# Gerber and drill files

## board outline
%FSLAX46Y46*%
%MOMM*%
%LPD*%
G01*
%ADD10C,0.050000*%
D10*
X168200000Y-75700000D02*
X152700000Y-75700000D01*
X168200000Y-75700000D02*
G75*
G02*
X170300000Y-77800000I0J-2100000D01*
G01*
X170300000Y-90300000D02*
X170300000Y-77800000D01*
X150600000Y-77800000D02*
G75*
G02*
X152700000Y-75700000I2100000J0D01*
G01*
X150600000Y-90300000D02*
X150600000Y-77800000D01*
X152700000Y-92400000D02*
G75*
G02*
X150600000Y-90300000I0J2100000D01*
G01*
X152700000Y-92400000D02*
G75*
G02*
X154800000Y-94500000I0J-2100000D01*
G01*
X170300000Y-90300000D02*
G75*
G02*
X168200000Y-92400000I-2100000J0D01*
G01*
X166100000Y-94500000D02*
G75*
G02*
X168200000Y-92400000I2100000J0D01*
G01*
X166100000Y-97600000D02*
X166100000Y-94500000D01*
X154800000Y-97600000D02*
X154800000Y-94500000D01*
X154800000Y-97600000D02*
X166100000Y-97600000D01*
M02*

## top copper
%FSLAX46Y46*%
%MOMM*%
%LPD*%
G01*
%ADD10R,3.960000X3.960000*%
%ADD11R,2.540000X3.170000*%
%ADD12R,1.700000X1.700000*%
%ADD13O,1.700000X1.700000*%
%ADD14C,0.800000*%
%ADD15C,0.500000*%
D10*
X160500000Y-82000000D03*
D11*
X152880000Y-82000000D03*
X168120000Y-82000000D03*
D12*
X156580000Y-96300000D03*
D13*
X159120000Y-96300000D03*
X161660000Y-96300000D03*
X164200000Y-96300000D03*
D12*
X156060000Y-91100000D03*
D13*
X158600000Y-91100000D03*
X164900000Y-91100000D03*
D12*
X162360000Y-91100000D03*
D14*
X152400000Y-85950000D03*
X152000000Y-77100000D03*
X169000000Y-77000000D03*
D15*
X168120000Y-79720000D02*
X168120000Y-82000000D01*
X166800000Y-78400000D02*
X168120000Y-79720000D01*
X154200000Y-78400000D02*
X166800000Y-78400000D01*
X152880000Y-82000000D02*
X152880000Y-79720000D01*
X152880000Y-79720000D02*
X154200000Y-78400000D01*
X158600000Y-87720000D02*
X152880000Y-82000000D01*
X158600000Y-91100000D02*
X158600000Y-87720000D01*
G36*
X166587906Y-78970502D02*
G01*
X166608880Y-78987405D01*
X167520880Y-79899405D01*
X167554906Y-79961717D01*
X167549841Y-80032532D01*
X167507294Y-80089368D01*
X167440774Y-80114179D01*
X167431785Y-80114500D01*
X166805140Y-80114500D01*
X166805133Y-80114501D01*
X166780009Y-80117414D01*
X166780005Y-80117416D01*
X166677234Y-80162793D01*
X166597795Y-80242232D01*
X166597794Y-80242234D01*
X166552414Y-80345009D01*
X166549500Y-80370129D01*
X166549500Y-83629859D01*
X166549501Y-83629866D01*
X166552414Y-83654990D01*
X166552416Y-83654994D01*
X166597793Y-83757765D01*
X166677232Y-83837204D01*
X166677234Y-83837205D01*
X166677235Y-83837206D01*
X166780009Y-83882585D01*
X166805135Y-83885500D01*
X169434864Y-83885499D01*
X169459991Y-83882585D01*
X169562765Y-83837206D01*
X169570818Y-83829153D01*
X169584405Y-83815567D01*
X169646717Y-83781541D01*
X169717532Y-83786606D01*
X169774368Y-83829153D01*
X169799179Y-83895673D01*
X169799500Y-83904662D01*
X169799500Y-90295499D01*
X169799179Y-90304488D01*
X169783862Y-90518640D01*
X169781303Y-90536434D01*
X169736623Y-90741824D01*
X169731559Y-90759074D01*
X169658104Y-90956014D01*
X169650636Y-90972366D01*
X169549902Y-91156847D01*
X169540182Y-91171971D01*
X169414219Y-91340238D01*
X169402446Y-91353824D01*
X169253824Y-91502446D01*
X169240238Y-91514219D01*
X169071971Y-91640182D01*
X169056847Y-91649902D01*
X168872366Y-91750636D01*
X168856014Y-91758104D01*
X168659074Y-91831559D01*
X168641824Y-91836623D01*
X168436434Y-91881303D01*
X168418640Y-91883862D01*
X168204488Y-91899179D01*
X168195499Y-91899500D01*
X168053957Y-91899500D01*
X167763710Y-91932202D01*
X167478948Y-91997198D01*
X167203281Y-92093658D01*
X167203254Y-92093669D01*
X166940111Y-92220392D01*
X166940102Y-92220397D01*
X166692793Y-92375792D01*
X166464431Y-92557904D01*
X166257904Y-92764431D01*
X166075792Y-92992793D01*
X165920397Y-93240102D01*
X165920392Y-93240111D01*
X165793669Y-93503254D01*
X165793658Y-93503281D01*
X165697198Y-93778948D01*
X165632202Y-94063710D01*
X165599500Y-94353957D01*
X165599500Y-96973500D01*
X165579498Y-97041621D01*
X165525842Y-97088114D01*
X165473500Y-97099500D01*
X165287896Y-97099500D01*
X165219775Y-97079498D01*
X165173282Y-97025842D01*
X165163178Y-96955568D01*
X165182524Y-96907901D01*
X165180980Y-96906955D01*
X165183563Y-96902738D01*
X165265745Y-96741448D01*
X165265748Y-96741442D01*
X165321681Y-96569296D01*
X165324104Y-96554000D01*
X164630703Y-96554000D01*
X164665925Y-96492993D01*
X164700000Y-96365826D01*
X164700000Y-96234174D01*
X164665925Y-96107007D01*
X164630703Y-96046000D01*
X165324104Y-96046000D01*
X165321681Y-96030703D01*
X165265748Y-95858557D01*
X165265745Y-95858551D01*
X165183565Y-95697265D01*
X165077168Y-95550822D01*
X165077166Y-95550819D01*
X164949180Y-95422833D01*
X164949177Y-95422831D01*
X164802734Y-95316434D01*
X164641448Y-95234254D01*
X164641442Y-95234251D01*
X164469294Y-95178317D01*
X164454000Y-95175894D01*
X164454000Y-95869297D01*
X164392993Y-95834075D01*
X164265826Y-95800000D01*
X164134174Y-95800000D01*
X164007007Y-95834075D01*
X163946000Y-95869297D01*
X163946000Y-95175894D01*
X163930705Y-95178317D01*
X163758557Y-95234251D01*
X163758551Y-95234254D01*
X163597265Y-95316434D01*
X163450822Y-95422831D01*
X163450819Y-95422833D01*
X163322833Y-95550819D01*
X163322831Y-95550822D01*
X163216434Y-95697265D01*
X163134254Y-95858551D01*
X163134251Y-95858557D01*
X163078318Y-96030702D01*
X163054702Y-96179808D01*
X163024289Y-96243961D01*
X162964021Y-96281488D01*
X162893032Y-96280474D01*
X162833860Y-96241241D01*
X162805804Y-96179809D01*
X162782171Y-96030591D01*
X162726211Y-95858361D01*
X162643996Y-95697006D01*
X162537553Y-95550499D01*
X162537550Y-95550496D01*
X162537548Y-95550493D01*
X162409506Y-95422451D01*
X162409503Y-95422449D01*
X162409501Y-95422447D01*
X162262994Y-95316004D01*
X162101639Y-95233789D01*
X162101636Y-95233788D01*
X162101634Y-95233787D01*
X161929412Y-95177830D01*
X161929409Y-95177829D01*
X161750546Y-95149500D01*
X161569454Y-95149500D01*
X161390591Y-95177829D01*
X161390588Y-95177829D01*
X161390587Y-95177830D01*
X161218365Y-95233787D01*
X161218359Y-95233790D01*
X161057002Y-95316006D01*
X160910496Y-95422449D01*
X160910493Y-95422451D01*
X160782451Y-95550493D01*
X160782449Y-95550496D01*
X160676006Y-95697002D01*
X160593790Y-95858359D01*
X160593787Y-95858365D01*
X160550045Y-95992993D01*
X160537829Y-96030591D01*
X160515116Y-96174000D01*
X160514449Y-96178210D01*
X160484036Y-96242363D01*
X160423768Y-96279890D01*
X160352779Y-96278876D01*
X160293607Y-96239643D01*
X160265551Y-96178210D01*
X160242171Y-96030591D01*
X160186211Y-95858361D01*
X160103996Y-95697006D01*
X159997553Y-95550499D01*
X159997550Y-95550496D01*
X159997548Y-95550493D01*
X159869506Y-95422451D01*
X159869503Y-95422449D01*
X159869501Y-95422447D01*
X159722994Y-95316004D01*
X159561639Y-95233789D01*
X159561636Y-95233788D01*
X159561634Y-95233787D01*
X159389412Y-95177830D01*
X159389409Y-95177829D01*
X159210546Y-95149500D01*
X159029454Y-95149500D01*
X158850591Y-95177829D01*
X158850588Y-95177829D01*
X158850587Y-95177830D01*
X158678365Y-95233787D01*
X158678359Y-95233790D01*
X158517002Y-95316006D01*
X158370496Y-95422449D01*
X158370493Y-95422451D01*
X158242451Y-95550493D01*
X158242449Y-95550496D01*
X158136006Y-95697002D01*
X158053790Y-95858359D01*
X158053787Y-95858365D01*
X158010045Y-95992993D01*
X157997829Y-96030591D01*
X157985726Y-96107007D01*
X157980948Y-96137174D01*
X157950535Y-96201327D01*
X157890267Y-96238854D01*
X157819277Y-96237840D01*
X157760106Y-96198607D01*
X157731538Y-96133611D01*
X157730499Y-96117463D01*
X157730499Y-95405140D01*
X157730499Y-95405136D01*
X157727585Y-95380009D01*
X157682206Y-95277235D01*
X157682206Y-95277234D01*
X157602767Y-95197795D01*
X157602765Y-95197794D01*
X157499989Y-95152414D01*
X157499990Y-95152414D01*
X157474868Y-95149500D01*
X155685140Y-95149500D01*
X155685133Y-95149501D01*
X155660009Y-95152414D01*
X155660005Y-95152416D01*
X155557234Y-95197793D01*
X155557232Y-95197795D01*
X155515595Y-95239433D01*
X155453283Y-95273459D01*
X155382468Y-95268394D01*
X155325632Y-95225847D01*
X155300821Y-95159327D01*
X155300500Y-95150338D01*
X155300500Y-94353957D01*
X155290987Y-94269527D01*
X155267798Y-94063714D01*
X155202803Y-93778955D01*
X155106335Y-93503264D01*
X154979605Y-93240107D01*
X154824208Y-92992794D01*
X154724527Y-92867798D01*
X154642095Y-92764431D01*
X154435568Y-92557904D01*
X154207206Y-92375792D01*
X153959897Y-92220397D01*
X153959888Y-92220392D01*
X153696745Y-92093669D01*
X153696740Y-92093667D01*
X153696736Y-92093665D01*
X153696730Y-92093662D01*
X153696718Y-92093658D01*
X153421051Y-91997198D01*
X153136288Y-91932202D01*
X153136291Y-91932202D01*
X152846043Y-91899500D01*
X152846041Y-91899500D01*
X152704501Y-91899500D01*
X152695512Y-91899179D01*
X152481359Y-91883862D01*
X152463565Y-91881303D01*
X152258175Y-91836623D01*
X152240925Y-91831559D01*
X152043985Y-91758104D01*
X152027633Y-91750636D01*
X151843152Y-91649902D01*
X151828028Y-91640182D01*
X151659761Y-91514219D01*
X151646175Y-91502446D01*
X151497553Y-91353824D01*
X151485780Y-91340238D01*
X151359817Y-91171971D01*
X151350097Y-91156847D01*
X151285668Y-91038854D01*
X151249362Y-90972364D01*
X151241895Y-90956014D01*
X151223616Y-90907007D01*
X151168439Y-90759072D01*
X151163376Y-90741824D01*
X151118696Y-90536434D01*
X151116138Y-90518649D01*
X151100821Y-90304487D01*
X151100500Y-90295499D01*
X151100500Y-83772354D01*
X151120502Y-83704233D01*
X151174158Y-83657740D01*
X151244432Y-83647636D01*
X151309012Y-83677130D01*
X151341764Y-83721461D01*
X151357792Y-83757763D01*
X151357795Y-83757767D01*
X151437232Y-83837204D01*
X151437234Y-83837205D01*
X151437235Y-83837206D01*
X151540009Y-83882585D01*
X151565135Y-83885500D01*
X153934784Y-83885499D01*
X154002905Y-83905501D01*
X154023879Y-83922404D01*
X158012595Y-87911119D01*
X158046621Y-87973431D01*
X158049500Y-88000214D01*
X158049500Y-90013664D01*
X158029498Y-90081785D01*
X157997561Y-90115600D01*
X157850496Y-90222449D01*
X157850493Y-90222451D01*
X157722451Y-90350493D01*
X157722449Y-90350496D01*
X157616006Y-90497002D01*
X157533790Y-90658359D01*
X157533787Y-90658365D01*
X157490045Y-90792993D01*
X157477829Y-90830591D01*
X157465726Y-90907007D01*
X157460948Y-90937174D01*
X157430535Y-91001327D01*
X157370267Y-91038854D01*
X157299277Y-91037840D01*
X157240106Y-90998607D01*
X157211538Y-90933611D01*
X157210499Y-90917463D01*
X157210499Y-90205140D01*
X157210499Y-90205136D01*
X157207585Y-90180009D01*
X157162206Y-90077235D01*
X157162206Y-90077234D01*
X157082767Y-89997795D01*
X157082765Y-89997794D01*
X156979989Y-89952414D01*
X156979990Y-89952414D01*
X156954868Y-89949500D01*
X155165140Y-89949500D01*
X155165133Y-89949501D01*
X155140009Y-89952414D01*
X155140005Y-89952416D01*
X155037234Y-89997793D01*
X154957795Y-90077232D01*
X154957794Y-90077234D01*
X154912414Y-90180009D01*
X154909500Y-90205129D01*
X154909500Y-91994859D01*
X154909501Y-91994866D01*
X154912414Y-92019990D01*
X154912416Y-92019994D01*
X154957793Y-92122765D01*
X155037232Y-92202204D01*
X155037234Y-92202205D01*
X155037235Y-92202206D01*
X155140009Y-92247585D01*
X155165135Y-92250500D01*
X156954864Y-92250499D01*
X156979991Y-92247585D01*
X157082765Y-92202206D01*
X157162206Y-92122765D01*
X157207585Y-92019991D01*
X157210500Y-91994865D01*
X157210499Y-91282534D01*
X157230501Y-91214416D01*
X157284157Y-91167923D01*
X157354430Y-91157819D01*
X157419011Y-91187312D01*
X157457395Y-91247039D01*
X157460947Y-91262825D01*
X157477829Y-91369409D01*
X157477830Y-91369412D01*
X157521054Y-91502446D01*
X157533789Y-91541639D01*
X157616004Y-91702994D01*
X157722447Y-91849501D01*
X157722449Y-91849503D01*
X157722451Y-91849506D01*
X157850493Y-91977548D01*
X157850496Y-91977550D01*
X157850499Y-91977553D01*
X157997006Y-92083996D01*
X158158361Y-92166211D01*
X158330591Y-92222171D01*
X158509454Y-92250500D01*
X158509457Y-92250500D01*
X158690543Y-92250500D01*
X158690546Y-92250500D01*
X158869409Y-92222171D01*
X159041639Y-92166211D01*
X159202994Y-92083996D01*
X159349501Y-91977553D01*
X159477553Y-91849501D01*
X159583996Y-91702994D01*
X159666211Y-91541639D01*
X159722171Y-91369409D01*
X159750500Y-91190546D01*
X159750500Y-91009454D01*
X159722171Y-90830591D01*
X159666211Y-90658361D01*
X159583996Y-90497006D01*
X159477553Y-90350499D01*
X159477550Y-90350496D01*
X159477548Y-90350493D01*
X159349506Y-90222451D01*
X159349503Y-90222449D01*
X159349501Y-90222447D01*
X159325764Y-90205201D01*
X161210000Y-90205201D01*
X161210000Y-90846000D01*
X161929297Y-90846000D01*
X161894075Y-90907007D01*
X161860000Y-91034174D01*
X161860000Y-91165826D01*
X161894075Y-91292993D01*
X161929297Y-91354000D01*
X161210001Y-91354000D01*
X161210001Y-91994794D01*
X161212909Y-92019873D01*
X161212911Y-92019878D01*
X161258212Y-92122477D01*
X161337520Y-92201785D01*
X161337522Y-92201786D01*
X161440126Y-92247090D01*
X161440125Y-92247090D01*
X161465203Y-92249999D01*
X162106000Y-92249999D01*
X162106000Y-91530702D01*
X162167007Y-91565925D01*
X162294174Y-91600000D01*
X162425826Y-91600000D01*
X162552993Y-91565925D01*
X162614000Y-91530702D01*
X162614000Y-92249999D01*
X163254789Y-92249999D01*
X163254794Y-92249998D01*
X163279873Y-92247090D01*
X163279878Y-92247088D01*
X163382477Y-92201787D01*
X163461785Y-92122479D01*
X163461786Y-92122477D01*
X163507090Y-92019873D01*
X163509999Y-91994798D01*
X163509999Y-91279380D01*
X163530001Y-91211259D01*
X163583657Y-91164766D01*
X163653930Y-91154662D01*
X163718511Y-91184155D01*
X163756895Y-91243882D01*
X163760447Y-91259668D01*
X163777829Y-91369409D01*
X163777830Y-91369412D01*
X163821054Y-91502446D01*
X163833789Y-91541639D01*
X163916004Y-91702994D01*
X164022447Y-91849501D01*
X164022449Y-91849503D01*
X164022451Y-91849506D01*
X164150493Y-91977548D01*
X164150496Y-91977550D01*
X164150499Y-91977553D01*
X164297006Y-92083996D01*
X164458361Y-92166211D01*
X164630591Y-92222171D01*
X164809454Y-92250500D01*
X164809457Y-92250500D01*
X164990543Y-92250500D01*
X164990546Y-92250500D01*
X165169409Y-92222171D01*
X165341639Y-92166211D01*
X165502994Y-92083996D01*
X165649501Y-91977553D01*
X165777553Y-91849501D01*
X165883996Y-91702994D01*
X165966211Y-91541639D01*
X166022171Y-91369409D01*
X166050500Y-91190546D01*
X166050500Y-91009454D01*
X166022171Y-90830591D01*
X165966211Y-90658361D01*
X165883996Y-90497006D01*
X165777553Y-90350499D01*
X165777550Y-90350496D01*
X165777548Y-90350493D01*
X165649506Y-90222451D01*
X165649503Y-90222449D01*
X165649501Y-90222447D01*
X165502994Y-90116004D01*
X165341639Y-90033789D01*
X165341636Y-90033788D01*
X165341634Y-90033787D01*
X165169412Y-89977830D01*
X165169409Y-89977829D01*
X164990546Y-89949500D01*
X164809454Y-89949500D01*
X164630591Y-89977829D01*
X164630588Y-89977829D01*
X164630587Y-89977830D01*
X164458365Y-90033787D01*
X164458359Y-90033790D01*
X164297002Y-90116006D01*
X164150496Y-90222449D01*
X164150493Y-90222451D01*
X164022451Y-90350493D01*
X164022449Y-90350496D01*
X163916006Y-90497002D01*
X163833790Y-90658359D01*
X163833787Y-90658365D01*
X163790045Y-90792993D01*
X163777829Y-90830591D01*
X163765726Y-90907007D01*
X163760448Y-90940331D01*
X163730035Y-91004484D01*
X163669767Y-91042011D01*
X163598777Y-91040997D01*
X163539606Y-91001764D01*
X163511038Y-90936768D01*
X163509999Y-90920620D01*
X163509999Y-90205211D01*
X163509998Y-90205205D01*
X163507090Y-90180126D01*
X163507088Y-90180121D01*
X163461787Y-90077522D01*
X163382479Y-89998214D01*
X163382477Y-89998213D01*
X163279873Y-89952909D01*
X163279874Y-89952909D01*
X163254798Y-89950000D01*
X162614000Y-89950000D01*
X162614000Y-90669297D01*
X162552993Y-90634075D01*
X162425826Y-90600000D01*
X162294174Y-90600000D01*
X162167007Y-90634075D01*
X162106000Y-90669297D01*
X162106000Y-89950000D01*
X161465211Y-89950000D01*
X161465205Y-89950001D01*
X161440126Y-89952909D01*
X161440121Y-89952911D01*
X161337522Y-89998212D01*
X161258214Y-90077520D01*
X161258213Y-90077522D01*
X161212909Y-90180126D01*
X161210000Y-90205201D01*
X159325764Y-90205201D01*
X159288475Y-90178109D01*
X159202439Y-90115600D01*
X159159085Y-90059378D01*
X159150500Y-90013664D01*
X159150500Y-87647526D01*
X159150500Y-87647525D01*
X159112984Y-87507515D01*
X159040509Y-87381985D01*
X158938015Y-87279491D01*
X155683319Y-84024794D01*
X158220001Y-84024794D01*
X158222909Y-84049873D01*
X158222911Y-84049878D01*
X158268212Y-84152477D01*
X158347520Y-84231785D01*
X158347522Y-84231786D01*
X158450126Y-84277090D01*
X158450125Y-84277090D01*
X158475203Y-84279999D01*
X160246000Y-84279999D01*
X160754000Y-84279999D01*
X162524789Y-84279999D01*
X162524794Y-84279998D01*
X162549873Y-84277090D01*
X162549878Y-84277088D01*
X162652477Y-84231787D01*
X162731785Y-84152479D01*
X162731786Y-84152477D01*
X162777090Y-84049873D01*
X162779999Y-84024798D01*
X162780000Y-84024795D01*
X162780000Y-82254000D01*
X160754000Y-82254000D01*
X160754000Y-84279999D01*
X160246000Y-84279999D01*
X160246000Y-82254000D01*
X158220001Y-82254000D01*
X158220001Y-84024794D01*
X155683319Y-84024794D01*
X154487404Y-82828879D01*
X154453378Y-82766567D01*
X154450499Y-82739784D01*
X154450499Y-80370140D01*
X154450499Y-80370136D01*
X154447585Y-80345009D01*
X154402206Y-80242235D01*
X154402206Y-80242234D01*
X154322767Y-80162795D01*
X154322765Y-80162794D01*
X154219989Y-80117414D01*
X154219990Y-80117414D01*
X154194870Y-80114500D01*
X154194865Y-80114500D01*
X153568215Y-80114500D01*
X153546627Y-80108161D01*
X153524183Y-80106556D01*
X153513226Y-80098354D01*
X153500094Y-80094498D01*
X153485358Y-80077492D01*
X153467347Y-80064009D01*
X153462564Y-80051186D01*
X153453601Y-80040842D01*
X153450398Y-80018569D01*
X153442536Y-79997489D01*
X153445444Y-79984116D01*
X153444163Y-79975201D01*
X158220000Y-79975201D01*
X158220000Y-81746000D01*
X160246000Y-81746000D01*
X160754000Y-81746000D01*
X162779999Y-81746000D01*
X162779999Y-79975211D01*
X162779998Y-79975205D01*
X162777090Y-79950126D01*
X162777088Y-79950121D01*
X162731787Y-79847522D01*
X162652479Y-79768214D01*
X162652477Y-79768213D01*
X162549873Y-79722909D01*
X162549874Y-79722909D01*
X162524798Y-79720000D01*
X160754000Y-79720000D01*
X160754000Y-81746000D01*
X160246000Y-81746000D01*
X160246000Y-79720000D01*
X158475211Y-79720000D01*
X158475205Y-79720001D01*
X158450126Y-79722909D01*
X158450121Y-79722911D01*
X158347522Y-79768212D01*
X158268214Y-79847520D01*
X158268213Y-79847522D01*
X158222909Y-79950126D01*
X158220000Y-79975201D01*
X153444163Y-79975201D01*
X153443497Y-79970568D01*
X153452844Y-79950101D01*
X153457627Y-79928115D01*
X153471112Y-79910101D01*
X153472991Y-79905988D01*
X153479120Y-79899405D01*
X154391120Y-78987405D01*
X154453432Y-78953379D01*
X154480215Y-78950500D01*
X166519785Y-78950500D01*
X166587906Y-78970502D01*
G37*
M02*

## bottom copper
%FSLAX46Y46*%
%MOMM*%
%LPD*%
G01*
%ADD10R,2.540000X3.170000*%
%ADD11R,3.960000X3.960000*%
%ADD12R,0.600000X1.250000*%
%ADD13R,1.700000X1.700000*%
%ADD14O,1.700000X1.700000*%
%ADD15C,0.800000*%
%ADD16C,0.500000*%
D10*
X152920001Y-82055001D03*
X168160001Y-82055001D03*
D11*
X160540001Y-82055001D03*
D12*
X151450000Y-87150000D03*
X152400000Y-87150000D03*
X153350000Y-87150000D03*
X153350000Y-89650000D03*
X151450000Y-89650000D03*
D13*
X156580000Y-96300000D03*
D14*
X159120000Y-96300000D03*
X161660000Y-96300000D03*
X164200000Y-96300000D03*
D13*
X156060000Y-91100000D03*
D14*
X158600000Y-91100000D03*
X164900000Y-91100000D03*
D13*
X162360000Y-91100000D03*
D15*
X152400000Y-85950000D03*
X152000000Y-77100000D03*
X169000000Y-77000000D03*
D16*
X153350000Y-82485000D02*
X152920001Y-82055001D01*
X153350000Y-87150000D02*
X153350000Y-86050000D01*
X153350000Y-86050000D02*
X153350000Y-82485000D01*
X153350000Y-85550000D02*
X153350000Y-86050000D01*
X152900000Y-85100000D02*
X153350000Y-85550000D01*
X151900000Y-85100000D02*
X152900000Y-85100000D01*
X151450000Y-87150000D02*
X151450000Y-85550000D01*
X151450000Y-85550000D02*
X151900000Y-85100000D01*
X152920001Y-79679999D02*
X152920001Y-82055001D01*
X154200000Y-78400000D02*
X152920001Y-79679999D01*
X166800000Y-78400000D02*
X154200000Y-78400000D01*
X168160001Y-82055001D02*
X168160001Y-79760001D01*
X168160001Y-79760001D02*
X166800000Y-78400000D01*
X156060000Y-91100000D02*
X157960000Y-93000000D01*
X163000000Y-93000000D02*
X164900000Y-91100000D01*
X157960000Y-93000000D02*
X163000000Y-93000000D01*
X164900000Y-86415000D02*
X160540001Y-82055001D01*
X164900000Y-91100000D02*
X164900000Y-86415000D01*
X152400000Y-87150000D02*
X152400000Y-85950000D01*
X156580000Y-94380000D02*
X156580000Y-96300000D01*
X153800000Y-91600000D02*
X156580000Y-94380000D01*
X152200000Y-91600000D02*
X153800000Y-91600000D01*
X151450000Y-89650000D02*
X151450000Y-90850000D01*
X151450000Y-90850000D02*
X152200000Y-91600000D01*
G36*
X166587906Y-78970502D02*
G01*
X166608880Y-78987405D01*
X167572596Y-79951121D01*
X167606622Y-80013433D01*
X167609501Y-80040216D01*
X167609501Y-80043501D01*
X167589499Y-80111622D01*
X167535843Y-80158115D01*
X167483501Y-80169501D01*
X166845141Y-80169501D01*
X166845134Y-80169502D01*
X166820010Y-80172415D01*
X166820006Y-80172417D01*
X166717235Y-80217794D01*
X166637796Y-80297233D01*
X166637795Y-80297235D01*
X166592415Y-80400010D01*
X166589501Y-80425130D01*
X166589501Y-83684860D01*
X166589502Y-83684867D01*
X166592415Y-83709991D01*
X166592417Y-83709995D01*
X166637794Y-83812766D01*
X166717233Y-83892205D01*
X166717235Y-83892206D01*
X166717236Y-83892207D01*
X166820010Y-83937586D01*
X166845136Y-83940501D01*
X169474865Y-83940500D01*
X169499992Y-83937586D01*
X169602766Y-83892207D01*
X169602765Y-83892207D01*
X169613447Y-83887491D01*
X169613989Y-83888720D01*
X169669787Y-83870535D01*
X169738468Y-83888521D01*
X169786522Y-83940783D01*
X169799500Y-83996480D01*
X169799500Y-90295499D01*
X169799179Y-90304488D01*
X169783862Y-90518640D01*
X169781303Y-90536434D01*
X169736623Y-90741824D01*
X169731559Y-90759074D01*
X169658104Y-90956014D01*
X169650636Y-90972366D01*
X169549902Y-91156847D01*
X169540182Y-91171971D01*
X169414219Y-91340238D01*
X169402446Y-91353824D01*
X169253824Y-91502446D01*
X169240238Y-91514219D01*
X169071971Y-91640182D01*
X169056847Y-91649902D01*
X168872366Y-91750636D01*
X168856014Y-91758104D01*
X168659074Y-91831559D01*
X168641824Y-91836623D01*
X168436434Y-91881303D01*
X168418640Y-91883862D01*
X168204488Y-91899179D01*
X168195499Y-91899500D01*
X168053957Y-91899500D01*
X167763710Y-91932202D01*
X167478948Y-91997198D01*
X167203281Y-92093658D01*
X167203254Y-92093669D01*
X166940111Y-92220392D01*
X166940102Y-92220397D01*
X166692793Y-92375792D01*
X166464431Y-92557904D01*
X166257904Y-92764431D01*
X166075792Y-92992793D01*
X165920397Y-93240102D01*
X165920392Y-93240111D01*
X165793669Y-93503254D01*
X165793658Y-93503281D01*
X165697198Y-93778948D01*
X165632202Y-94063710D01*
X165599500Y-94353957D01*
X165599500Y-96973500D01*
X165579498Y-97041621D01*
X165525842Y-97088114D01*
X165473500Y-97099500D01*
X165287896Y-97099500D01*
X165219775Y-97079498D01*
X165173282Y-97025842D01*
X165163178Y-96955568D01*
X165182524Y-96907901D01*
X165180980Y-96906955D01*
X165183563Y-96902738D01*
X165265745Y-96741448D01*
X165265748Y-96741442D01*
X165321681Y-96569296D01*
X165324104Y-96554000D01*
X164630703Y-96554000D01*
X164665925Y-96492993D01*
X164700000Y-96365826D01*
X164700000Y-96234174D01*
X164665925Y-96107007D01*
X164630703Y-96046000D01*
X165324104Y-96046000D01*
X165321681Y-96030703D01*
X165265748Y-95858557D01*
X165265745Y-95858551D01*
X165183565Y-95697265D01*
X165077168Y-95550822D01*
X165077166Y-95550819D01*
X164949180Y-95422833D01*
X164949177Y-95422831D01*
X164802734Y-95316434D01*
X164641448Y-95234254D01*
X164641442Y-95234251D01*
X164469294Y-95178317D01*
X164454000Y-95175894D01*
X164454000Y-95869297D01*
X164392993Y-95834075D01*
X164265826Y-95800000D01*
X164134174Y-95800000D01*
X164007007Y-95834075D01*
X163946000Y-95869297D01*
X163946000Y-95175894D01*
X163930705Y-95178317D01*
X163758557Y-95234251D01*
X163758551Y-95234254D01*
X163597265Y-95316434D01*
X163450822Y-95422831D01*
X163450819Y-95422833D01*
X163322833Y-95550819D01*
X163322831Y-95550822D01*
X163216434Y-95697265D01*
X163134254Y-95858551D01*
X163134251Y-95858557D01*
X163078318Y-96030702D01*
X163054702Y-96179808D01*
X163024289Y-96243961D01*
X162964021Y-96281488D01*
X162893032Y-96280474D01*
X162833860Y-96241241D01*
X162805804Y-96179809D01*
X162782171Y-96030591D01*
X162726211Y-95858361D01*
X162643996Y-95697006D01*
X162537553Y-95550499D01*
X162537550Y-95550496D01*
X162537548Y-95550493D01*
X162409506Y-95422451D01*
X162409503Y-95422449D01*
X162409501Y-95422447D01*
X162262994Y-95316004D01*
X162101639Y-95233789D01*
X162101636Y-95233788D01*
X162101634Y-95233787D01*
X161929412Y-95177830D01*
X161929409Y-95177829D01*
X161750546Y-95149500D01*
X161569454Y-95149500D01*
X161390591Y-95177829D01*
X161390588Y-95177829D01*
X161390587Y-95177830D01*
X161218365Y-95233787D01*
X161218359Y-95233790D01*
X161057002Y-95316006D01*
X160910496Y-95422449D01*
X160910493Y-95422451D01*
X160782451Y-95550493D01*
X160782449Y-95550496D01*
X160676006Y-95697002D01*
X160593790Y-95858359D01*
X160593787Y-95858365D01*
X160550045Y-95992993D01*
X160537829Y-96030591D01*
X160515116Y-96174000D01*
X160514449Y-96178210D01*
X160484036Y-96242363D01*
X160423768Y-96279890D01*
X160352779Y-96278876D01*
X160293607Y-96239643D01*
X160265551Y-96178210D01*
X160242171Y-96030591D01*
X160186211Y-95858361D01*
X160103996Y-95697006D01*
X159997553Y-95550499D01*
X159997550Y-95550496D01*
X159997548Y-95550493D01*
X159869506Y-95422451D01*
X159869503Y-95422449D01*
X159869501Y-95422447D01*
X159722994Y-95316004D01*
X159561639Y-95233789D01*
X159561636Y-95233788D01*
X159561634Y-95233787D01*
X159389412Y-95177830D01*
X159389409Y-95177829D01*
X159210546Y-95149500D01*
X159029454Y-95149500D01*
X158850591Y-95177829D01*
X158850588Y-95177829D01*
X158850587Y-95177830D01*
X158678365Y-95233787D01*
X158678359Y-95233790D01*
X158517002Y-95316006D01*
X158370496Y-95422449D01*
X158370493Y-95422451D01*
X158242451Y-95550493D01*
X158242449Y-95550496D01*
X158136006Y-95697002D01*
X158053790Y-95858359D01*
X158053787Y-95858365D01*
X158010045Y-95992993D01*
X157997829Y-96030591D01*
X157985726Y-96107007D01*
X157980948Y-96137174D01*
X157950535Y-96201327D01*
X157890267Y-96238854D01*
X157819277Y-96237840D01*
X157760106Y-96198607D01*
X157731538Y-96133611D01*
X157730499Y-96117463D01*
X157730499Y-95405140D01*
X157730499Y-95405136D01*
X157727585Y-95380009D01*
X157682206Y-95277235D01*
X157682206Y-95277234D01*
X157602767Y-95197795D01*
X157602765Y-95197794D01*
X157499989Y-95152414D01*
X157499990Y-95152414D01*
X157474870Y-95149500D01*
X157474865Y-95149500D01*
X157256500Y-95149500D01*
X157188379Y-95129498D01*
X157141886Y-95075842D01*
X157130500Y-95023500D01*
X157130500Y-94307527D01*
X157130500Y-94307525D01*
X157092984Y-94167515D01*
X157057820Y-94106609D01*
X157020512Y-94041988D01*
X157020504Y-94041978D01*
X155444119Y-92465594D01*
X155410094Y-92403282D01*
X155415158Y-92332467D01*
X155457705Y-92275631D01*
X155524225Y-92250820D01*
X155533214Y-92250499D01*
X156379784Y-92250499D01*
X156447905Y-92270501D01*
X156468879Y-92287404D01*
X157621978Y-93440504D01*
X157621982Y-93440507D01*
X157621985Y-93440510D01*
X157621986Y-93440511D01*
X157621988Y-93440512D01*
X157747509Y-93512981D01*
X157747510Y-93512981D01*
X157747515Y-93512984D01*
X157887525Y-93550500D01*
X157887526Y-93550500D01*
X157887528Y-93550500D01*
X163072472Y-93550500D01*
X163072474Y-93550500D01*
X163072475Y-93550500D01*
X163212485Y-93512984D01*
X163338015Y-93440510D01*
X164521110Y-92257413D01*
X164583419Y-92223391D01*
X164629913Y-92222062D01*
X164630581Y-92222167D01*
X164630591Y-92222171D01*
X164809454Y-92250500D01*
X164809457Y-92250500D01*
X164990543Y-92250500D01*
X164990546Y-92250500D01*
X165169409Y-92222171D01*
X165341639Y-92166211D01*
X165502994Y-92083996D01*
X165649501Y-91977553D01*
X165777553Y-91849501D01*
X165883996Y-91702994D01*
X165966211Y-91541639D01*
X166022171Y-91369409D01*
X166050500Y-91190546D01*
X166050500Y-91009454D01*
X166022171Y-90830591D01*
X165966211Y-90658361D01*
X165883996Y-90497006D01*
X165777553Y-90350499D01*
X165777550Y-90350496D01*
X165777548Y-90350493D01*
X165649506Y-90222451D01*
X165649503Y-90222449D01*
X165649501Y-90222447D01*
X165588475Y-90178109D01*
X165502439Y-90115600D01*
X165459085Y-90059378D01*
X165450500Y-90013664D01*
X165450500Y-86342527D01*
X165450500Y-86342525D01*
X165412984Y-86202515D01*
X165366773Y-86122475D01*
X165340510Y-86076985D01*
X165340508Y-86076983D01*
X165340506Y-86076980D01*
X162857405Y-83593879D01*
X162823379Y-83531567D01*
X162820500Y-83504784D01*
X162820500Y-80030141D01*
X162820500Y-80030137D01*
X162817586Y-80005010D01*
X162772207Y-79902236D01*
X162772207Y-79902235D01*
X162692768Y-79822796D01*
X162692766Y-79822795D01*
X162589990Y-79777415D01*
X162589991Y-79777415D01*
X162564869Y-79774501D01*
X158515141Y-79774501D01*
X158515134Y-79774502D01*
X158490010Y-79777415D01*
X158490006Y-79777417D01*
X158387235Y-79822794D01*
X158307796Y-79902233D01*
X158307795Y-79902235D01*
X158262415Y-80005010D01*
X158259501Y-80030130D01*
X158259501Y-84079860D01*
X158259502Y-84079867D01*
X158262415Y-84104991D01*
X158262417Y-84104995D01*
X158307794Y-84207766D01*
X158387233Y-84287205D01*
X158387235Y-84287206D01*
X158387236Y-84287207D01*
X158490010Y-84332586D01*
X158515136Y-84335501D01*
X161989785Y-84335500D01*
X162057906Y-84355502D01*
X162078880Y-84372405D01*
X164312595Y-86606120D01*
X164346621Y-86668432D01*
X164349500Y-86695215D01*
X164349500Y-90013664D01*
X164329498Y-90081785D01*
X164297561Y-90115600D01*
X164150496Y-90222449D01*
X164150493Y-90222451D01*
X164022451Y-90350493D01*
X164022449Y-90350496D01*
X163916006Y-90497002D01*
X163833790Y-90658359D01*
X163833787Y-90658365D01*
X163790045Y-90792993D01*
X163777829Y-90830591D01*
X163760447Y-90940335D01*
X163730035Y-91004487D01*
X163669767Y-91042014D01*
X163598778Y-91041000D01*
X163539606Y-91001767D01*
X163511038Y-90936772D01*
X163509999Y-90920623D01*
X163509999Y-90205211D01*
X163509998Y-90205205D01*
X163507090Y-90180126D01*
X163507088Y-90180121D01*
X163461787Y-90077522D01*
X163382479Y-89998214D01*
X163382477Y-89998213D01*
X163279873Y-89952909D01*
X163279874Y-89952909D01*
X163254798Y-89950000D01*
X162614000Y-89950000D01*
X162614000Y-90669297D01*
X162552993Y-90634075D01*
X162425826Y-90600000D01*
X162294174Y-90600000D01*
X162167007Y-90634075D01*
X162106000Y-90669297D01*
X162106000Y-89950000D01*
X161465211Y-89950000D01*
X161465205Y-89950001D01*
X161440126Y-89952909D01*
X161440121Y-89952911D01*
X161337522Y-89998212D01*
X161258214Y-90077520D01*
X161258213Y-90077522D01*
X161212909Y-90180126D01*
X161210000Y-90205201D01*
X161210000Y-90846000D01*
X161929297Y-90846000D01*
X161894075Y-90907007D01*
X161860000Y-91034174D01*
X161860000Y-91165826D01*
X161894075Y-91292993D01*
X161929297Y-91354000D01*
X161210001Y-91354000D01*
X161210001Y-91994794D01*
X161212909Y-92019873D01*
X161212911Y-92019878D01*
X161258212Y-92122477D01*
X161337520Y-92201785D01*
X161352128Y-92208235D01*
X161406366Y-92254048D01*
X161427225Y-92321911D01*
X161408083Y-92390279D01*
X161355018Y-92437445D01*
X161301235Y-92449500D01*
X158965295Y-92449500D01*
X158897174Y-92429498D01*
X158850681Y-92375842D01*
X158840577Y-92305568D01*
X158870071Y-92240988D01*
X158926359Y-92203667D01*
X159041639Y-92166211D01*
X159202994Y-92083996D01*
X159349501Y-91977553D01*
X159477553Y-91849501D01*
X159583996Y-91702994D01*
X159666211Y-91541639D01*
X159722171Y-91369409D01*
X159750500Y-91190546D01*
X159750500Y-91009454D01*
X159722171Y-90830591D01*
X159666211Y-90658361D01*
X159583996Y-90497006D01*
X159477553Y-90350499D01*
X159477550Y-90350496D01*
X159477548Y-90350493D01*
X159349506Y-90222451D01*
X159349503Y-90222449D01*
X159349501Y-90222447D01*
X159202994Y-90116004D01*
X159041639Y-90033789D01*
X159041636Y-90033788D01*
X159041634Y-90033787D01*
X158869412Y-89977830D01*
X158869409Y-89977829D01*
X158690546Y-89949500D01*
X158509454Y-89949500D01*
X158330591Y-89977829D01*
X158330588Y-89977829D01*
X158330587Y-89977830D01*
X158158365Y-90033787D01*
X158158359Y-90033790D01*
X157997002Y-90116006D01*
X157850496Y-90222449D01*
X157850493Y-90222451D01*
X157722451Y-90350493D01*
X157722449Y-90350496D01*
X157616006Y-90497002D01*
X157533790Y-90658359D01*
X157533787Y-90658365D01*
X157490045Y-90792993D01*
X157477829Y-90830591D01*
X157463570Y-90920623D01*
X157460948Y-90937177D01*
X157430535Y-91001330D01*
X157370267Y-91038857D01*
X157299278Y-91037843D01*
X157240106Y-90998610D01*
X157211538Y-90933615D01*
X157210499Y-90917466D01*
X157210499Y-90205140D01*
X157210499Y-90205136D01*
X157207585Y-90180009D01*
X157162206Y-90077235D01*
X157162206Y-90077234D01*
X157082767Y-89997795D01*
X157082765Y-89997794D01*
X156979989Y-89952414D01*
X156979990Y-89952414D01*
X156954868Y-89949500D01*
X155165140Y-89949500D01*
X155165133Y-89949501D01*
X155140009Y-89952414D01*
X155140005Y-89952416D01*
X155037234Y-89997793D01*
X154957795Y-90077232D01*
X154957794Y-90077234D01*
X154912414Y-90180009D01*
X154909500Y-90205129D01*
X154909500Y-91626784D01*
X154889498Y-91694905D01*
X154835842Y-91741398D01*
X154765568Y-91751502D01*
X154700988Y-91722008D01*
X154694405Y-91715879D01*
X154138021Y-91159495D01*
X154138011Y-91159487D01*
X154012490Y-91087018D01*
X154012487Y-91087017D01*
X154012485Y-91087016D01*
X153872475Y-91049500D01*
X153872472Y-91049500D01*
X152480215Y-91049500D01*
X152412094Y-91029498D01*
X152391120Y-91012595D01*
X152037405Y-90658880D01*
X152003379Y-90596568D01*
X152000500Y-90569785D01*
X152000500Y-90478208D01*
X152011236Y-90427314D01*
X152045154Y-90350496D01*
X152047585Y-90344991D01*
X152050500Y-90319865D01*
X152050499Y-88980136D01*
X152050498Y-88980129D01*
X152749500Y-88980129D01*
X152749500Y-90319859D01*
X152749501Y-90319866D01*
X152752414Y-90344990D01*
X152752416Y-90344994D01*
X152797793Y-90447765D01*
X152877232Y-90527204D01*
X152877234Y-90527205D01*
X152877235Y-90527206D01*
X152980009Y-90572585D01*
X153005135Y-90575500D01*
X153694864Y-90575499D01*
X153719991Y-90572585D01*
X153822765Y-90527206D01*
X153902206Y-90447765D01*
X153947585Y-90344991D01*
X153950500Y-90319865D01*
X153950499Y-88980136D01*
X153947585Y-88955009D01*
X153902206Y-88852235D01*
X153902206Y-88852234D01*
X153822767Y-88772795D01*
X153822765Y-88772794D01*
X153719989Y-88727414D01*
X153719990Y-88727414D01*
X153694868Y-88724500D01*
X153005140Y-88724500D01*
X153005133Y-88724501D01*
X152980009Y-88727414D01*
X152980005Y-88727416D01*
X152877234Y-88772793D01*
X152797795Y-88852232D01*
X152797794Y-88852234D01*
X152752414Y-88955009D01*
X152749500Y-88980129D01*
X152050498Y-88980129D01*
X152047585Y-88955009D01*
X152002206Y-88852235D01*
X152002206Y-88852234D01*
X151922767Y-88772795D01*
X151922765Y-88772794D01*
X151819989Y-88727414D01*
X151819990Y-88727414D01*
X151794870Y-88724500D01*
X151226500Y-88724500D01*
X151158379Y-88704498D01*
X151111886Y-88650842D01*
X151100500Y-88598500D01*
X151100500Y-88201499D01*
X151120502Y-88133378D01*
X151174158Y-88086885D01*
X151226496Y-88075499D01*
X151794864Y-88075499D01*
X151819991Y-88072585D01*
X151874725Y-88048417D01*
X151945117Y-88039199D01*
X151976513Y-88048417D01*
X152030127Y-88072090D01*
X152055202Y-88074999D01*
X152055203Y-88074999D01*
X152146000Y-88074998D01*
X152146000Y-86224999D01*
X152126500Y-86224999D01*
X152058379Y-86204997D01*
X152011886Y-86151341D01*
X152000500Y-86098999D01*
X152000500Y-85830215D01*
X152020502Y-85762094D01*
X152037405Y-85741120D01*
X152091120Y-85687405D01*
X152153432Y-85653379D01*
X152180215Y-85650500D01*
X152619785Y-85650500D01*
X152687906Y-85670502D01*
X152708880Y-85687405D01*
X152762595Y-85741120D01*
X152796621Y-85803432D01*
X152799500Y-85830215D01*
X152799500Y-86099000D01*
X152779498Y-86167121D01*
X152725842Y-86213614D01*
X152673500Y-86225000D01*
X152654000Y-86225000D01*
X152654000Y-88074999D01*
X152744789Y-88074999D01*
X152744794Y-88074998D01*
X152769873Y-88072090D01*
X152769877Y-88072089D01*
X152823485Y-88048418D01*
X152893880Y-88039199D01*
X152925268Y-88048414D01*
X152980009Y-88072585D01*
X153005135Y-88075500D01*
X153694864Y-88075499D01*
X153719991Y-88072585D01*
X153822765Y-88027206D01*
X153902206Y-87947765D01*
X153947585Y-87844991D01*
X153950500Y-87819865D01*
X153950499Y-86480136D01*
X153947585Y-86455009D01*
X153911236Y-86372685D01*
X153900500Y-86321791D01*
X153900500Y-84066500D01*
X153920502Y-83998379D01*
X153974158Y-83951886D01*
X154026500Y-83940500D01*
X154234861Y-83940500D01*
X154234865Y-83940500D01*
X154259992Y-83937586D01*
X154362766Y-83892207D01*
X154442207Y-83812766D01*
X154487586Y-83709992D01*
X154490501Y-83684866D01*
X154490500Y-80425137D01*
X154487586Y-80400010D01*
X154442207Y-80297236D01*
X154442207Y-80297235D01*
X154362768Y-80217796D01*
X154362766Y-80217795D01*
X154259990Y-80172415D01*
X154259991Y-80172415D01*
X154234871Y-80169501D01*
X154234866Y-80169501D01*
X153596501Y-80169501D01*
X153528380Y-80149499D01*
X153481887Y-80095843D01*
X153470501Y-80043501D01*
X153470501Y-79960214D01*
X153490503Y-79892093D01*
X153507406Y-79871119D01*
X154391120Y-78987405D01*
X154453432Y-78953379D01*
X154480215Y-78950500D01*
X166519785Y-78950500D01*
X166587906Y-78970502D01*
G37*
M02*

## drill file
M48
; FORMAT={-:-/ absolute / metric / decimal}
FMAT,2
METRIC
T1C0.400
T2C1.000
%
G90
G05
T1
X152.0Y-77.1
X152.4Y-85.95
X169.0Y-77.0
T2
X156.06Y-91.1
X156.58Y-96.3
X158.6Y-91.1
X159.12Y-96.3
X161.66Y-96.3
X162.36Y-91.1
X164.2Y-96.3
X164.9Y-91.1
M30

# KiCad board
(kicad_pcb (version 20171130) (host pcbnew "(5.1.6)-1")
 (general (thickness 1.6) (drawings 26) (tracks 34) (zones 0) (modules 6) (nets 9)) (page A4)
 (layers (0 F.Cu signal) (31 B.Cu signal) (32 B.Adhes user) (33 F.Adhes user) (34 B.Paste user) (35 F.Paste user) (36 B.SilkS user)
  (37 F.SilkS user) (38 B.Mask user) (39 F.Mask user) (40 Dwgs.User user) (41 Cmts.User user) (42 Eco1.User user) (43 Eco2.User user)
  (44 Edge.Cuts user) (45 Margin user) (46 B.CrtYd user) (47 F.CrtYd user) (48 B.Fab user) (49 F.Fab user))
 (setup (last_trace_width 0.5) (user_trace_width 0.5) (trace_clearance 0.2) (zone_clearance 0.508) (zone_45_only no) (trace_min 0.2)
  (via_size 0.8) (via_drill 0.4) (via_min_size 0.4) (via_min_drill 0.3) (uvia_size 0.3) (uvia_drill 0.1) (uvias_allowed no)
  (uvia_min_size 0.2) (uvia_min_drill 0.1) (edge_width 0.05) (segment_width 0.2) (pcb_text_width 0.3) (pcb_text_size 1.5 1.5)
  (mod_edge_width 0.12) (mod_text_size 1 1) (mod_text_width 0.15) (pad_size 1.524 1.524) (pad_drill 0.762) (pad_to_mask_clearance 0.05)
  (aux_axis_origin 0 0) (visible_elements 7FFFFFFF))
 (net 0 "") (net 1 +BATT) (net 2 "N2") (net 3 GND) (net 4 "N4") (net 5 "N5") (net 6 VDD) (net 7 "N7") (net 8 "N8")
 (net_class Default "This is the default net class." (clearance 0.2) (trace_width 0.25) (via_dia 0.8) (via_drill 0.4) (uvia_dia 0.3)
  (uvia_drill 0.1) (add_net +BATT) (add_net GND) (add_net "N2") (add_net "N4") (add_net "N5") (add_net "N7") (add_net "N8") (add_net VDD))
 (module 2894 (layer B.Cu) (at 160.540001 82.055001)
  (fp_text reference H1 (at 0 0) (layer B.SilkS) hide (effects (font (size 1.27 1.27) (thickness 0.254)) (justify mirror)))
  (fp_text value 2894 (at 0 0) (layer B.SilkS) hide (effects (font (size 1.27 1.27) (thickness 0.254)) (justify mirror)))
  (pad 1 smd rect (at -7.62 0) (size 2.54 3.17) (layers B.Cu B.Paste B.Mask) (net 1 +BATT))
  (pad 2 smd rect (at 7.62 0) (size 2.54 3.17) (layers B.Cu B.Paste B.Mask) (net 1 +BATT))
  (pad MP1 smd rect (at 0 0) (size 3.96 3.96) (layers B.Cu B.Paste B.Mask) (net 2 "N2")))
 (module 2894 (layer F.Cu) (at 160.5 82 180)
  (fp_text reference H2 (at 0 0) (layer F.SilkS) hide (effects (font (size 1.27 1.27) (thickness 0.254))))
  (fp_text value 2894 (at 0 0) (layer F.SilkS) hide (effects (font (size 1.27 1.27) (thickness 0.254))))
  (pad MP1 smd rect (at 0 0 180) (size 3.96 3.96) (layers F.Cu F.Paste F.Mask) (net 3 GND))
  (pad 2 smd rect (at 7.62 0 180) (size 2.54 3.17) (layers F.Cu F.Paste F.Mask) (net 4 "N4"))
  (pad 1 smd rect (at -7.62 0 180) (size 2.54 3.17) (layers F.Cu F.Paste F.Mask) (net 4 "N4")))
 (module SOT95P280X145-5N (layer B.Cu) (at 152.4 88.4 270)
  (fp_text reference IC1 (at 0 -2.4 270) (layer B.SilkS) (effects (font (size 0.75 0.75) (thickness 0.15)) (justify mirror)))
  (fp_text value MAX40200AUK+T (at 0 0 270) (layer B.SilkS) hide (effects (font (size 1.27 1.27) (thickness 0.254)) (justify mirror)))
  (pad 1 smd rect (at -1.25 0.95 180) (size 0.6 1.25) (layers B.Cu B.Paste B.Mask) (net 1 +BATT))
  (pad 2 smd rect (at -1.25 0 180) (size 0.6 1.25) (layers B.Cu B.Paste B.Mask) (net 3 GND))
  (pad 3 smd rect (at -1.25 -0.95 180) (size 0.6 1.25) (layers B.Cu B.Paste B.Mask) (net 1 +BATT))
  (pad 4 smd rect (at 1.25 -0.95 180) (size 0.6 1.25) (layers B.Cu B.Paste B.Mask) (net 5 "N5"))
  (pad 5 smd rect (at 1.25 0.95 180) (size 0.6 1.25) (layers B.Cu B.Paste B.Mask) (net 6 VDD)))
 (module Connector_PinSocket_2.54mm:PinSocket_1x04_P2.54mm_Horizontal (layer F.Cu) (at 156.58 96.3 90)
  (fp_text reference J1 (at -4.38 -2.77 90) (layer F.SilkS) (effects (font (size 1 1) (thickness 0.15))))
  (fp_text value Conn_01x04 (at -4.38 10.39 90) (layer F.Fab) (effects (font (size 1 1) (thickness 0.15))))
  (pad 1 thru_hole rect (at 0 0 90) (size 1.7 1.7) (drill 1) (layers *.Cu *.Mask) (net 6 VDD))
  (pad 2 thru_hole oval (at 0 2.54 90) (size 1.7 1.7) (drill 1) (layers *.Cu *.Mask) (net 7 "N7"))
  (pad 3 thru_hole oval (at 0 5.08 90) (size 1.7 1.7) (drill 1) (layers *.Cu *.Mask) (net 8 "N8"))
  (pad 4 thru_hole oval (at 0 7.62 90) (size 1.7 1.7) (drill 1) (layers *.Cu *.Mask) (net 3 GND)))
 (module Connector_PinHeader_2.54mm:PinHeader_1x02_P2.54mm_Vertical (layer F.Cu) (at 156.06 91.1 90)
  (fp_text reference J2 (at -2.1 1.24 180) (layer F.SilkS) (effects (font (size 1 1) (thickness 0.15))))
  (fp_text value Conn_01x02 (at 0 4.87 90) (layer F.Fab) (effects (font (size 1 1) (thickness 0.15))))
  (pad 1 thru_hole rect (at 0 0 90) (size 1.7 1.7) (drill 1) (layers *.Cu *.Mask) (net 2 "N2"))
  (pad 2 thru_hole oval (at 0 2.54 90) (size 1.7 1.7) (drill 1) (layers *.Cu *.Mask) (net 4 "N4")))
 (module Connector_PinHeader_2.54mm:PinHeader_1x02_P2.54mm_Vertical (layer F.Cu) (at 162.36 91.1 90)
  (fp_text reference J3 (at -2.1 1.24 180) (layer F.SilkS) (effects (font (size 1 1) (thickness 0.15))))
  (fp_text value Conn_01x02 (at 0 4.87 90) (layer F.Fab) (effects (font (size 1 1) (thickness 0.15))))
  (pad 2 thru_hole oval (at 0 2.54 90) (size 1.7 1.7) (drill 1) (layers *.Cu *.Mask) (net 2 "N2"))
  (pad 1 thru_hole rect (at 0 0 90) (size 1.7 1.7) (drill 1) (layers *.Cu *.Mask) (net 3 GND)))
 (gr_line (start 168.2 75.7) (end 152.7 75.7) (layer Edge.Cuts) (width 0.05))
 (gr_arc (start 168.2 77.8) (end 170.3 77.8) (angle -90) (layer Edge.Cuts) (width 0.05))
 (gr_line (start 170.3 90.3) (end 170.3 77.8) (layer Edge.Cuts) (width 0.05))
 (gr_arc (start 152.7 77.8) (end 152.7 75.7) (angle -90) (layer Edge.Cuts) (width 0.05))
 (gr_line (start 150.6 90.3) (end 150.6 77.8) (layer Edge.Cuts) (width 0.05))
 (gr_arc (start 152.7 90.3) (end 150.6 90.3) (angle -90) (layer Edge.Cuts) (width 0.05))
 (gr_arc (start 152.7 94.5) (end 154.8 94.5) (angle -90) (layer Edge.Cuts) (width 0.05))
 (gr_arc (start 168.2 90.3) (end 168.2 92.4) (angle -90) (layer Edge.Cuts) (width 0.05))
 (gr_arc (start 168.2 94.5) (end 168.2 92.4) (angle -90) (layer Edge.Cuts) (width 0.05))
 (gr_line (start 166.1 97.6) (end 166.1 94.5) (layer Edge.Cuts) (width 0.05))
 (gr_line (start 154.8 97.6) (end 154.8 94.5) (layer Edge.Cuts) (width 0.05))
 (gr_line (start 154.8 97.6) (end 166.1 97.6) (layer Edge.Cuts) (width 0.05))
 (segment (start 153.35 82.485) (end 152.920001 82.055001) (width 0.5) (layer B.Cu) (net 1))
 (segment (start 153.35 87.15) (end 153.35 86.05) (width 0.5) (layer B.Cu) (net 1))
 (segment (start 153.35 86.05) (end 153.35 82.485) (width 0.5) (layer B.Cu) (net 1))
 (segment (start 153.35 85.55) (end 153.35 86.05) (width 0.5) (layer B.Cu) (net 1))
 (segment (start 152.9 85.1) (end 153.35 85.55) (width 0.5) (layer B.Cu) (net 1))
 (segment (start 151.9 85.1) (end 152.9 85.1) (width 0.5) (layer B.Cu) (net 1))
 (segment (start 151.45 87.15) (end 151.45 85.55) (width 0.5) (layer B.Cu) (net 1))
 (segment (start 151.45 85.55) (end 151.9 85.1) (width 0.5) (layer B.Cu) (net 1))
 (segment (start 152.920001 79.679999) (end 152.920001 82.055001) (width 0.5) (layer B.Cu) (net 1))
 (segment (start 154.2 78.4) (end 152.920001 79.679999) (width 0.5) (layer B.Cu) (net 1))
 (segment (start 166.8 78.4) (end 154.2 78.4) (width 0.5) (layer B.Cu) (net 1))
 (segment (start 168.160001 82.055001) (end 168.160001 79.760001) (width 0.5) (layer B.Cu) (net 1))
 (segment (start 168.160001 79.760001) (end 166.8 78.4) (width 0.5) (layer B.Cu) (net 1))
 (segment (start 156.06 91.1) (end 157.96 93) (width 0.5) (layer B.Cu) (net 2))
 (segment (start 163 93) (end 164.9 91.1) (width 0.5) (layer B.Cu) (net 2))
 (segment (start 157.96 93) (end 163 93) (width 0.5) (layer B.Cu) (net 2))
 (segment (start 164.9 86.415) (end 160.540001 82.055001) (width 0.5) (layer B.Cu) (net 2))
 (segment (start 164.9 91.1) (end 164.9 86.415) (width 0.5) (layer B.Cu) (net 2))
 (via (at 152.4 85.95) (size 0.8) (drill 0.4) (layers F.Cu B.Cu) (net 3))
 (segment (start 152.4 87.15) (end 152.4 85.95) (width 0.5) (layer B.Cu) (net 3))
 (via (at 152 77.1) (size 0.8) (drill 0.4) (layers F.Cu B.Cu) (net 3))
 (via (at 169 77) (size 0.8) (drill 0.4) (layers F.Cu B.Cu) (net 3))
 (segment (start 168.12 79.72) (end 168.12 82) (width 0.5) (layer F.Cu) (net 4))
 (segment (start 166.8 78.4) (end 168.12 79.72) (width 0.5) (layer F.Cu) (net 4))
 (segment (start 154.2 78.4) (end 166.8 78.4) (width 0.5) (layer F.Cu) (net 4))
 (segment (start 152.88 82) (end 152.88 79.72) (width 0.5) (layer F.Cu) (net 4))
 (segment (start 152.88 79.72) (end 154.2 78.4) (width 0.5) (layer F.Cu) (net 4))
 (segment (start 158.6 87.72) (end 152.88 82) (width 0.5) (layer F.Cu) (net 4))
 (segment (start 158.6 91.1) (end 158.6 87.72) (width 0.5) (layer F.Cu) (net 4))
 (segment (start 156.58 94.38) (end 156.58 96.3) (width 0.5) (layer B.Cu) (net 6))
 (segment (start 153.8 91.6) (end 156.58 94.38) (width 0.5) (layer B.Cu) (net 6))
 (segment (start 152.2 91.6) (end 153.8 91.6) (width 0.5) (layer B.Cu) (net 6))
 (segment (start 151.45 89.65) (end 151.45 90.85) (width 0.5) (layer B.Cu) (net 6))
 (segment (start 151.45 90.85) (end 152.2 91.6) (width 0.5) (layer B.Cu) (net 6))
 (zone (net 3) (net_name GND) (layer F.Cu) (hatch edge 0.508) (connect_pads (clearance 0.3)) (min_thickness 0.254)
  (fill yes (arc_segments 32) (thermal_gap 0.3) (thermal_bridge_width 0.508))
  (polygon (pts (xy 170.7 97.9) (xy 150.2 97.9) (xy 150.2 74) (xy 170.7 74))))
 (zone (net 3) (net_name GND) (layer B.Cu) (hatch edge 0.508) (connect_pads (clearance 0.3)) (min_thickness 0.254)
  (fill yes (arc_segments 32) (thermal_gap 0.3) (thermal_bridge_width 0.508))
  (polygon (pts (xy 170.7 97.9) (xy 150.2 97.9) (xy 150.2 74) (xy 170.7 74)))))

